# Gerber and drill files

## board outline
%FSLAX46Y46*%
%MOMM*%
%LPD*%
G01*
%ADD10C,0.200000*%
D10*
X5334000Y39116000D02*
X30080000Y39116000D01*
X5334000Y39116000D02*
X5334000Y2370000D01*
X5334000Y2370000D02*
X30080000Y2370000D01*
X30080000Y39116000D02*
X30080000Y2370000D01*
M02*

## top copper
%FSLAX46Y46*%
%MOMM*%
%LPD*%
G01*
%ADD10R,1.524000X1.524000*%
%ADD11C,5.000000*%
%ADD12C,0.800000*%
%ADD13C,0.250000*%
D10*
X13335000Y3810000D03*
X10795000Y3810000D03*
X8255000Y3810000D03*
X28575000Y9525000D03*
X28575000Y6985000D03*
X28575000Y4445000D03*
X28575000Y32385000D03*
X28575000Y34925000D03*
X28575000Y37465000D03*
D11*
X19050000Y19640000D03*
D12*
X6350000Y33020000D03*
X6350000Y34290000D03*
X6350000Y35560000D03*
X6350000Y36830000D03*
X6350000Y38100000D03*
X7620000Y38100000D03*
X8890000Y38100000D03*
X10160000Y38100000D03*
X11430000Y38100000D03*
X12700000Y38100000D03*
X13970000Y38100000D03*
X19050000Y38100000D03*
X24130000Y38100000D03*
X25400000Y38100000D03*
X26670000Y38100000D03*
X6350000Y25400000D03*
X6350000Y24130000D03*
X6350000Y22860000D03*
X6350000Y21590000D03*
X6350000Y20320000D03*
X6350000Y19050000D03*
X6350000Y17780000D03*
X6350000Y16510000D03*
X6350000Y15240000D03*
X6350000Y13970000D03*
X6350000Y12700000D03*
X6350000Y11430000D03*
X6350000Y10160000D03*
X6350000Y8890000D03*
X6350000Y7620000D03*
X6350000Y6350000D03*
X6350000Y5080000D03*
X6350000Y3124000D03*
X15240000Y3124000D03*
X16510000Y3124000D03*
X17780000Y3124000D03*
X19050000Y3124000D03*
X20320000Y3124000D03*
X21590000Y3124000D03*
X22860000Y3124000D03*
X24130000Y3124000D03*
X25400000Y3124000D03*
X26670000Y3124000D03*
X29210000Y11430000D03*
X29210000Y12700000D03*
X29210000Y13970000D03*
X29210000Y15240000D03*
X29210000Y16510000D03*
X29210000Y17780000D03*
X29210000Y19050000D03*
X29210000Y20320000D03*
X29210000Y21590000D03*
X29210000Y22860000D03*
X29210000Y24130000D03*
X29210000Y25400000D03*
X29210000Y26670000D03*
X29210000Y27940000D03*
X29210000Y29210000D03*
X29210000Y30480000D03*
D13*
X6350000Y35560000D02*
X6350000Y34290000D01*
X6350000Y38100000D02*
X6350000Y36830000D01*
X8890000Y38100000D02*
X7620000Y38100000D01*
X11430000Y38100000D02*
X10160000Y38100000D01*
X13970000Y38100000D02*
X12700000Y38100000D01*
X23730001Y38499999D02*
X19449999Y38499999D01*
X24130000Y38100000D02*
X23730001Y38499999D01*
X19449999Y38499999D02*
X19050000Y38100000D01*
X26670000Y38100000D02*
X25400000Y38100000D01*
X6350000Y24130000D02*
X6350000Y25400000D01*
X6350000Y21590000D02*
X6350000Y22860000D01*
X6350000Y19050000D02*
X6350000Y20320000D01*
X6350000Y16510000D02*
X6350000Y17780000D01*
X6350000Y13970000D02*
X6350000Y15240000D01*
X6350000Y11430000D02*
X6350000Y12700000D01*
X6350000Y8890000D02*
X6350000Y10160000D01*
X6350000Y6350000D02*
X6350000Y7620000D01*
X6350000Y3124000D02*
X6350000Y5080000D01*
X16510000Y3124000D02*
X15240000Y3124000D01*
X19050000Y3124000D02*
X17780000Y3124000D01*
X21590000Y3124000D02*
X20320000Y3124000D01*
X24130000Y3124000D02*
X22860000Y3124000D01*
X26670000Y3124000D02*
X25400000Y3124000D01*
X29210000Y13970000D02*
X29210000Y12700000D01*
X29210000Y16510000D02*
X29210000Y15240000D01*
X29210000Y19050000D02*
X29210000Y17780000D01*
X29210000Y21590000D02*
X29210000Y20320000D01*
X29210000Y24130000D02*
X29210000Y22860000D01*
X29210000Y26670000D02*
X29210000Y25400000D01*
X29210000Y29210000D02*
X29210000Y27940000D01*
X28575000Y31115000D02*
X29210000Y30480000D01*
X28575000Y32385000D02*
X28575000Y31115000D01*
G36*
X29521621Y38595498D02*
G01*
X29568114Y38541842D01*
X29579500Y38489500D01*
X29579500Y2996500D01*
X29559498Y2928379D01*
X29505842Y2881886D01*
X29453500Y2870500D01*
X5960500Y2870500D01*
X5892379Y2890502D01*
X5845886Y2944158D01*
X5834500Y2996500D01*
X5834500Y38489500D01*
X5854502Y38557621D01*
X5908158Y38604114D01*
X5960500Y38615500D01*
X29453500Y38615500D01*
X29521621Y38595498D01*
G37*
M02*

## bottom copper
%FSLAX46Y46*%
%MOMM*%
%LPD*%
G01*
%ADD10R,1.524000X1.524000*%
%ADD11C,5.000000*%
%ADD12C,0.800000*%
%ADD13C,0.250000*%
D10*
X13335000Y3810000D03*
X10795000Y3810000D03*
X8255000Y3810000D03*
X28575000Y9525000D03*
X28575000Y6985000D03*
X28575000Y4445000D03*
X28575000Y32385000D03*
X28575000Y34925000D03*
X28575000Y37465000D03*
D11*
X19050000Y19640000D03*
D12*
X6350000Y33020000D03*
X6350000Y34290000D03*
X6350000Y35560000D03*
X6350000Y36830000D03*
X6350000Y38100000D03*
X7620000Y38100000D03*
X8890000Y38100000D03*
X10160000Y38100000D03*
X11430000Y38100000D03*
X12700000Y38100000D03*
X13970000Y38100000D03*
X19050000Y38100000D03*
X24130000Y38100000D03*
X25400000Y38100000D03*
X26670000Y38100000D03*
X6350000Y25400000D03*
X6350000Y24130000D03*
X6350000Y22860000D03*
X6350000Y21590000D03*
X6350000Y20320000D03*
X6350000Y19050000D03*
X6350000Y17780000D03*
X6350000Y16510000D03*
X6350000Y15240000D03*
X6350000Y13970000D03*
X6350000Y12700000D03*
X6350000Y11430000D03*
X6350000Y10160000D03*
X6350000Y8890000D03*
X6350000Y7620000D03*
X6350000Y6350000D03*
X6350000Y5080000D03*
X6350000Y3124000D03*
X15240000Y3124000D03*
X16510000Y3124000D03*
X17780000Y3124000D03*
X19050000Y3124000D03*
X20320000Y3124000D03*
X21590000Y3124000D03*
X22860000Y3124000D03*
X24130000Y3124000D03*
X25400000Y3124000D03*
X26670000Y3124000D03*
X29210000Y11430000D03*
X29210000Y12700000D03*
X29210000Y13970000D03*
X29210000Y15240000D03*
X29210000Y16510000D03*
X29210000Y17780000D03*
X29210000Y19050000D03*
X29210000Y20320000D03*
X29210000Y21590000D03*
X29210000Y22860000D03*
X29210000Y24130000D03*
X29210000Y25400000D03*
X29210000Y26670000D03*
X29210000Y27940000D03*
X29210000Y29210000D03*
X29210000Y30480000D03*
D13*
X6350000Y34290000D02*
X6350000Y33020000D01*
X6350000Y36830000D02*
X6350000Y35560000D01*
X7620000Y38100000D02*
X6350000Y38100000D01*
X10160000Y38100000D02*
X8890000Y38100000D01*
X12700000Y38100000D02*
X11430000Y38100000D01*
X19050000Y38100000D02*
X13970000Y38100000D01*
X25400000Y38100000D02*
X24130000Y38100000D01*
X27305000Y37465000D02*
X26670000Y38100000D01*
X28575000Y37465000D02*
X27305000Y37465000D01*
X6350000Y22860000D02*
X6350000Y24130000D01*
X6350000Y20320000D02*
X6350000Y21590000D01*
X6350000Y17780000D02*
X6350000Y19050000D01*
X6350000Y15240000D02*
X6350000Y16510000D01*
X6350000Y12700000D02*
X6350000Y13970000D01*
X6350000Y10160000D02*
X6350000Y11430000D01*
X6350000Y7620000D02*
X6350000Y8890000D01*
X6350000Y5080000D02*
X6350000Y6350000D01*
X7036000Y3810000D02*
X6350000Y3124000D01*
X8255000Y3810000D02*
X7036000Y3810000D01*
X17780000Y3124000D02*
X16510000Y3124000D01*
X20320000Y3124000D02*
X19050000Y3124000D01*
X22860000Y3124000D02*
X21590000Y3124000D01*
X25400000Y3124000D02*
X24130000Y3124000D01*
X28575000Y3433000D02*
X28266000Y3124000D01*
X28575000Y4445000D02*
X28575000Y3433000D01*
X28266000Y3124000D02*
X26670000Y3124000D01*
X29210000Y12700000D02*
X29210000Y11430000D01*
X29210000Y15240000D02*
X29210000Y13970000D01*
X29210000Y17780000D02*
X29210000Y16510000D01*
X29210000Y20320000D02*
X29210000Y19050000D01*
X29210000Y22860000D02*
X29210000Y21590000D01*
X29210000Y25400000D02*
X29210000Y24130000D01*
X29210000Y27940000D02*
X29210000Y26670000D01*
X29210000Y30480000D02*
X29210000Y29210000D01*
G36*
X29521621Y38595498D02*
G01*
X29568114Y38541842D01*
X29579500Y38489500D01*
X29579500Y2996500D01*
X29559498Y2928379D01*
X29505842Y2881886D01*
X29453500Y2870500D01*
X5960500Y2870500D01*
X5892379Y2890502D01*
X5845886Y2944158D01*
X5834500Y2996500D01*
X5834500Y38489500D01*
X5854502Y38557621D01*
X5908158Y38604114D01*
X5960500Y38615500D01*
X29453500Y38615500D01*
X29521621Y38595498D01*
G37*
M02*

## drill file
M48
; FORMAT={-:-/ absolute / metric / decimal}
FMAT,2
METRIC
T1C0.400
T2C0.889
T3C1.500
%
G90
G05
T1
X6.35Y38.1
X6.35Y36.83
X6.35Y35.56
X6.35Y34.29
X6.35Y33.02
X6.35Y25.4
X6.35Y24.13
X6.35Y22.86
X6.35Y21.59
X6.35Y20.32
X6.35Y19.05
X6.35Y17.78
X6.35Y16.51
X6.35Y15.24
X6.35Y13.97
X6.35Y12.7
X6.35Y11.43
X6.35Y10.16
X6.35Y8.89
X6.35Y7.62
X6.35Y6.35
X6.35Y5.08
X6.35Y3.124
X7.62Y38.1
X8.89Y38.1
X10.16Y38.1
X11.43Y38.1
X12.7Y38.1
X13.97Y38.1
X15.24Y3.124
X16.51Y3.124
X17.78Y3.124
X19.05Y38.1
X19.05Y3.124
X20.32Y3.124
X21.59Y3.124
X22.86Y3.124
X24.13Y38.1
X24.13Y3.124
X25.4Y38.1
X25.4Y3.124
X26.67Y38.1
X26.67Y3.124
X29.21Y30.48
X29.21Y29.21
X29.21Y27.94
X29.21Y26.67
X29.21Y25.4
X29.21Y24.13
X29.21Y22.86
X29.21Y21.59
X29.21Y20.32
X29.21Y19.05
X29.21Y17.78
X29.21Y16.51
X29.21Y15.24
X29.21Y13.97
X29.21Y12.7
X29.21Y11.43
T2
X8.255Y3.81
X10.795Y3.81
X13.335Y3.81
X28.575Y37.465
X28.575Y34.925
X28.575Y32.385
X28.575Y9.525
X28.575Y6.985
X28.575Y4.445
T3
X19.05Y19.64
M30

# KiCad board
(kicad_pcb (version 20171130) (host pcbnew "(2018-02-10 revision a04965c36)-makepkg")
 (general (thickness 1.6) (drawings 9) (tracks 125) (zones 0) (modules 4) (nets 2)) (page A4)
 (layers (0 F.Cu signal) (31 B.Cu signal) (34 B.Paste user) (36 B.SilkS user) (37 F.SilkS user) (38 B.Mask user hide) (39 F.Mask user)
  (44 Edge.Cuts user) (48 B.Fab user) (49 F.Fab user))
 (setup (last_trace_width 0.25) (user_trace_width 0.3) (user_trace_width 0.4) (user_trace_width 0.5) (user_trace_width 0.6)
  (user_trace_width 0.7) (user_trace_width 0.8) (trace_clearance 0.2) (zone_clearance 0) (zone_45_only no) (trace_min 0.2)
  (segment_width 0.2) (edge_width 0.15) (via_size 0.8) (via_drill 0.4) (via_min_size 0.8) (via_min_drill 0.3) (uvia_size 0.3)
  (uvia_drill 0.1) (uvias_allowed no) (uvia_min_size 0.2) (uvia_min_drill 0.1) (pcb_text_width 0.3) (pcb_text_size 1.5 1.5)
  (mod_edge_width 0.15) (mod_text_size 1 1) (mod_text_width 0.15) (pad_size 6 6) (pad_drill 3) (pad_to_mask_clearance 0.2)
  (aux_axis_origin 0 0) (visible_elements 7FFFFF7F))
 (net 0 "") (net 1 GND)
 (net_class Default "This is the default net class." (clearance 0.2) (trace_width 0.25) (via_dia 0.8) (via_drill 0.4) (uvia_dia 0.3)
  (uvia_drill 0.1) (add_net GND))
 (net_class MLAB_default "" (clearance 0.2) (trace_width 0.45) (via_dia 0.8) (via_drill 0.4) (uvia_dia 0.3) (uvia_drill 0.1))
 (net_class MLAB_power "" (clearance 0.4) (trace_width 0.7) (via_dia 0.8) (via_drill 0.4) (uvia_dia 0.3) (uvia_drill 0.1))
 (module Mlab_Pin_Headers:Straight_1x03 (layer F.Cu) (at 10.795 -3.81 90)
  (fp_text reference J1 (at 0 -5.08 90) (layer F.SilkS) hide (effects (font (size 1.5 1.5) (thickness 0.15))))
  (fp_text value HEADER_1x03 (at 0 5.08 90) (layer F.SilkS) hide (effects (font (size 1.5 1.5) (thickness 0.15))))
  (pad 3 thru_hole rect (at 0 2.54 90) (size 1.524 1.524) (drill 0.889) (layers *.Cu *.Mask F.SilkS) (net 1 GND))
  (pad 2 thru_hole rect (at 0 0 90) (size 1.524 1.524) (drill 0.889) (layers *.Cu *.Mask F.SilkS) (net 1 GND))
  (pad 1 thru_hole rect (at 0 -2.54 90) (size 1.524 1.524) (drill 0.889) (layers *.Cu *.Mask F.SilkS) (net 1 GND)))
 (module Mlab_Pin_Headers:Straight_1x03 (layer F.Cu) (at 28.575 -6.985)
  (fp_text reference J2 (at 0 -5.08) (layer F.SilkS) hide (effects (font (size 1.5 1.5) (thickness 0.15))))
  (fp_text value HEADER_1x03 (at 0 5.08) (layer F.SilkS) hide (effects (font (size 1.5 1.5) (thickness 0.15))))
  (pad 1 thru_hole rect (at 0 -2.54) (size 1.524 1.524) (drill 0.889) (layers *.Cu *.Mask F.SilkS) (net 1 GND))
  (pad 2 thru_hole rect (at 0 0) (size 1.524 1.524) (drill 0.889) (layers *.Cu *.Mask F.SilkS) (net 1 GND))
  (pad 3 thru_hole rect (at 0 2.54) (size 1.524 1.524) (drill 0.889) (layers *.Cu *.Mask F.SilkS) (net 1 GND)))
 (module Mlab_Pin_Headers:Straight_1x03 (layer F.Cu) (at 28.575 -34.925)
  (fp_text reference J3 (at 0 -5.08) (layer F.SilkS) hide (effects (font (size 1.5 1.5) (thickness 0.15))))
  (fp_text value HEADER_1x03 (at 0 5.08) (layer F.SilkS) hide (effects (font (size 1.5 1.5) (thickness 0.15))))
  (pad 3 thru_hole rect (at 0 2.54) (size 1.524 1.524) (drill 0.889) (layers *.Cu *.Mask F.SilkS) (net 1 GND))
  (pad 2 thru_hole rect (at 0 0) (size 1.524 1.524) (drill 0.889) (layers *.Cu *.Mask F.SilkS) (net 1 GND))
  (pad 1 thru_hole rect (at 0 -2.54) (size 1.524 1.524) (drill 0.889) (layers *.Cu *.Mask F.SilkS) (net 1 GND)))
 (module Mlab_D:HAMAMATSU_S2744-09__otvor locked (layer F.Cu) (at 19.05 -5.2 270)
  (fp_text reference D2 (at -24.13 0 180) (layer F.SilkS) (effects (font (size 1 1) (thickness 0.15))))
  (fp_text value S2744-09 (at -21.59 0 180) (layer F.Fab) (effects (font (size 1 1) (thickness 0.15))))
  (pad 1 thru_hole circle (at -14.44 0 270) (size 5 5) (drill 1.5) (layers *.Cu *.Mask) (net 1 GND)))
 (gr_line (start 5.334 -39.116) (end 30.08 -39.116) (layer Edge.Cuts) (width 0.2))
 (gr_line (start 5.334 -39.116) (end 5.334 -2.37) (layer Edge.Cuts) (width 0.2))
 (gr_line (start 5.334 -2.37) (end 30.08 -2.37) (layer Edge.Cuts) (width 0.2))
 (gr_line (start 30.08 -39.116) (end 30.08 -2.37) (layer Edge.Cuts) (width 0.2))
 (segment (start 6.35 -34.29) (end 6.35 -33.02) (width 0.25) (layer B.Cu) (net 1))
 (via (at 6.35 -33.02) (size 0.8) (drill 0.4) (layers F.Cu B.Cu) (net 1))
 (segment (start 6.35 -35.56) (end 6.35 -34.29) (width 0.25) (layer F.Cu) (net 1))
 (via (at 6.35 -34.29) (size 0.8) (drill 0.4) (layers F.Cu B.Cu) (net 1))
 (segment (start 6.35 -36.83) (end 6.35 -35.56) (width 0.25) (layer B.Cu) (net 1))
 (via (at 6.35 -35.56) (size 0.8) (drill 0.4) (layers F.Cu B.Cu) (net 1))
 (segment (start 6.35 -38.1) (end 6.35 -36.83) (width 0.25) (layer F.Cu) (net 1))
 (via (at 6.35 -36.83) (size 0.8) (drill 0.4) (layers F.Cu B.Cu) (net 1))
 (segment (start 7.62 -38.1) (end 6.35 -38.1) (width 0.25) (layer B.Cu) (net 1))
 (via (at 6.35 -38.1) (size 0.8) (drill 0.4) (layers F.Cu B.Cu) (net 1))
 (segment (start 8.89 -38.1) (end 7.62 -38.1) (width 0.25) (layer F.Cu) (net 1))
 (via (at 7.62 -38.1) (size 0.8) (drill 0.4) (layers F.Cu B.Cu) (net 1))
 (segment (start 10.16 -38.1) (end 8.89 -38.1) (width 0.25) (layer B.Cu) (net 1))
 (via (at 8.89 -38.1) (size 0.8) (drill 0.4) (layers F.Cu B.Cu) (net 1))
 (segment (start 11.43 -38.1) (end 10.16 -38.1) (width 0.25) (layer F.Cu) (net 1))
 (via (at 10.16 -38.1) (size 0.8) (drill 0.4) (layers F.Cu B.Cu) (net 1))
 (segment (start 12.7 -38.1) (end 11.43 -38.1) (width 0.25) (layer B.Cu) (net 1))
 (via (at 11.43 -38.1) (size 0.8) (drill 0.4) (layers F.Cu B.Cu) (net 1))
 (segment (start 13.97 -38.1) (end 12.7 -38.1) (width 0.25) (layer F.Cu) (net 1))
 (via (at 12.7 -38.1) (size 0.8) (drill 0.4) (layers F.Cu B.Cu) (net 1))
 (segment (start 19.05 -38.1) (end 13.97 -38.1) (width 0.25) (layer B.Cu) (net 1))
 (via (at 13.97 -38.1) (size 0.8) (drill 0.4) (layers F.Cu B.Cu) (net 1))
 (segment (start 23.730001 -38.499999) (end 19.449999 -38.499999) (width 0.25) (layer F.Cu) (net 1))
 (segment (start 24.13 -38.1) (end 23.730001 -38.499999) (width 0.25) (layer F.Cu) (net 1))
 (segment (start 19.449999 -38.499999) (end 19.05 -38.1) (width 0.25) (layer F.Cu) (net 1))
 (via (at 19.05 -38.1) (size 0.8) (drill 0.4) (layers F.Cu B.Cu) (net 1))
 (segment (start 25.4 -38.1) (end 24.13 -38.1) (width 0.25) (layer B.Cu) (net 1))
 (via (at 24.13 -38.1) (size 0.8) (drill 0.4) (layers F.Cu B.Cu) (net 1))
 (segment (start 26.67 -38.1) (end 25.4 -38.1) (width 0.25) (layer F.Cu) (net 1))
 (via (at 25.4 -38.1) (size 0.8) (drill 0.4) (layers F.Cu B.Cu) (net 1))
 (segment (start 27.305 -37.465) (end 26.67 -38.1) (width 0.25) (layer B.Cu) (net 1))
 (segment (start 28.575 -37.465) (end 27.305 -37.465) (width 0.25) (layer B.Cu) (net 1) (status 10))
 (via (at 26.67 -38.1) (size 0.8) (drill 0.4) (layers F.Cu B.Cu) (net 1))
 (segment (start 6.35 -24.13) (end 6.35 -25.4) (width 0.25) (layer F.Cu) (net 1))
 (via (at 6.35 -25.4) (size 0.8) (drill 0.4) (layers F.Cu B.Cu) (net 1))
 (segment (start 6.35 -22.86) (end 6.35 -24.13) (width 0.25) (layer B.Cu) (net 1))
 (via (at 6.35 -24.13) (size 0.8) (drill 0.4) (layers F.Cu B.Cu) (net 1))
 (segment (start 6.35 -21.59) (end 6.35 -22.86) (width 0.25) (layer F.Cu) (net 1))
 (via (at 6.35 -22.86) (size 0.8) (drill 0.4) (layers F.Cu B.Cu) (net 1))
 (segment (start 6.35 -20.32) (end 6.35 -21.59) (width 0.25) (layer B.Cu) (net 1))
 (via (at 6.35 -21.59) (size 0.8) (drill 0.4) (layers F.Cu B.Cu) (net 1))
 (segment (start 6.35 -19.05) (end 6.35 -20.32) (width 0.25) (layer F.Cu) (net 1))
 (via (at 6.35 -20.32) (size 0.8) (drill 0.4) (layers F.Cu B.Cu) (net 1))
 (segment (start 6.35 -17.78) (end 6.35 -19.05) (width 0.25) (layer B.Cu) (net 1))
 (via (at 6.35 -19.05) (size 0.8) (drill 0.4) (layers F.Cu B.Cu) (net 1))
 (segment (start 6.35 -16.51) (end 6.35 -17.78) (width 0.25) (layer F.Cu) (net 1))
 (via (at 6.35 -17.78) (size 0.8) (drill 0.4) (layers F.Cu B.Cu) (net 1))
 (segment (start 6.35 -15.24) (end 6.35 -16.51) (width 0.25) (layer B.Cu) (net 1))
 (via (at 6.35 -16.51) (size 0.8) (drill 0.4) (layers F.Cu B.Cu) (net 1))
 (segment (start 6.35 -13.97) (end 6.35 -15.24) (width 0.25) (layer F.Cu) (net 1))
 (via (at 6.35 -15.24) (size 0.8) (drill 0.4) (layers F.Cu B.Cu) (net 1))
 (segment (start 6.35 -12.7) (end 6.35 -13.97) (width 0.25) (layer B.Cu) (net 1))
 (via (at 6.35 -13.97) (size 0.8) (drill 0.4) (layers F.Cu B.Cu) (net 1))
 (segment (start 6.35 -11.43) (end 6.35 -12.7) (width 0.25) (layer F.Cu) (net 1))
 (via (at 6.35 -12.7) (size 0.8) (drill 0.4) (layers F.Cu B.Cu) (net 1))
 (segment (start 6.35 -10.16) (end 6.35 -11.43) (width 0.25) (layer B.Cu) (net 1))
 (via (at 6.35 -11.43) (size 0.8) (drill 0.4) (layers F.Cu B.Cu) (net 1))
 (segment (start 6.35 -8.89) (end 6.35 -10.16) (width 0.25) (layer F.Cu) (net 1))
 (via (at 6.35 -10.16) (size 0.8) (drill 0.4) (layers F.Cu B.Cu) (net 1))
 (segment (start 6.35 -7.62) (end 6.35 -8.89) (width 0.25) (layer B.Cu) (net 1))
 (via (at 6.35 -8.89) (size 0.8) (drill 0.4) (layers F.Cu B.Cu) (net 1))
 (segment (start 6.35 -6.35) (end 6.35 -7.62) (width 0.25) (layer F.Cu) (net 1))
 (via (at 6.35 -7.62) (size 0.8) (drill 0.4) (layers F.Cu B.Cu) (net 1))
 (segment (start 6.35 -5.08) (end 6.35 -6.35) (width 0.25) (layer B.Cu) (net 1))
 (via (at 6.35 -6.35) (size 0.8) (drill 0.4) (layers F.Cu B.Cu) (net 1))
 (segment (start 6.35 -3.124) (end 6.35 -5.08) (width 0.25) (layer F.Cu) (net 1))
 (via (at 6.35 -5.08) (size 0.8) (drill 0.4) (layers F.Cu B.Cu) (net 1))
 (segment (start 7.036 -3.81) (end 6.35 -3.124) (width 0.25) (layer B.Cu) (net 1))
 (segment (start 8.255 -3.81) (end 7.036 -3.81) (width 0.25) (layer B.Cu) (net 1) (status 10))
 (via (at 6.35 -3.124) (size 0.8) (drill 0.4) (layers F.Cu B.Cu) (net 1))
 (segment (start 16.51 -3.124) (end 15.24 -3.124) (width 0.25) (layer F.Cu) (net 1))
 (via (at 15.24 -3.124) (size 0.8) (drill 0.4) (layers F.Cu B.Cu) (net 1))
 (segment (start 17.78 -3.124) (end 16.51 -3.124) (width 0.25) (layer B.Cu) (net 1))
 (via (at 16.51 -3.124) (size 0.8) (drill 0.4) (layers F.Cu B.Cu) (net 1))
 (segment (start 19.05 -3.124) (end 17.78 -3.124) (width 0.25) (layer F.Cu) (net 1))
 (via (at 17.78 -3.124) (size 0.8) (drill 0.4) (layers F.Cu B.Cu) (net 1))
 (segment (start 20.32 -3.124) (end 19.05 -3.124) (width 0.25) (layer B.Cu) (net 1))
 (via (at 19.05 -3.124) (size 0.8) (drill 0.4) (layers F.Cu B.Cu) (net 1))
 (segment (start 21.59 -3.124) (end 20.32 -3.124) (width 0.25) (layer F.Cu) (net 1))
 (via (at 20.32 -3.124) (size 0.8) (drill 0.4) (layers F.Cu B.Cu) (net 1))
 (segment (start 22.86 -3.124) (end 21.59 -3.124) (width 0.25) (layer B.Cu) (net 1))
 (via (at 21.59 -3.124) (size 0.8) (drill 0.4) (layers F.Cu B.Cu) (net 1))
 (segment (start 24.13 -3.124) (end 22.86 -3.124) (width 0.25) (layer F.Cu) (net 1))
 (via (at 22.86 -3.124) (size 0.8) (drill 0.4) (layers F.Cu B.Cu) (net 1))
 (segment (start 25.4 -3.124) (end 24.13 -3.124) (width 0.25) (layer B.Cu) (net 1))
 (via (at 24.13 -3.124) (size 0.8) (drill 0.4) (layers F.Cu B.Cu) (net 1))
 (segment (start 26.67 -3.124) (end 25.4 -3.124) (width 0.25) (layer F.Cu) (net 1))
 (via (at 25.4 -3.124) (size 0.8) (drill 0.4) (layers F.Cu B.Cu) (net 1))
 (segment (start 28.575 -3.433) (end 28.266 -3.124) (width 0.25) (layer B.Cu) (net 1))
 (segment (start 28.575 -4.445) (end 28.575 -3.433) (width 0.25) (layer B.Cu) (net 1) (status 10))
 (segment (start 28.266 -3.124) (end 26.67 -3.124) (width 0.25) (layer B.Cu) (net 1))
 (via (at 26.67 -3.124) (size 0.8) (drill 0.4) (layers F.Cu B.Cu) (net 1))
 (via (at 29.21 -11.43) (size 0.8) (drill 0.4) (layers F.Cu B.Cu) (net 1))
 (segment (start 29.21 -12.7) (end 29.21 -11.43) (width 0.25) (layer B.Cu) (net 1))
 (segment (start 29.21 -13.97) (end 29.21 -12.7) (width 0.25) (layer F.Cu) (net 1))
 (via (at 29.21 -12.7) (size 0.8) (drill 0.4) (layers F.Cu B.Cu) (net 1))
 (segment (start 29.21 -15.24) (end 29.21 -13.97) (width 0.25) (layer B.Cu) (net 1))
 (via (at 29.21 -13.97) (size 0.8) (drill 0.4) (layers F.Cu B.Cu) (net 1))
 (segment (start 29.21 -16.51) (end 29.21 -15.24) (width 0.25) (layer F.Cu) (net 1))
 (via (at 29.21 -15.24) (size 0.8) (drill 0.4) (layers F.Cu B.Cu) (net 1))
 (segment (start 29.21 -17.78) (end 29.21 -16.51) (width 0.25) (layer B.Cu) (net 1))
 (via (at 29.21 -16.51) (size 0.8) (drill 0.4) (layers F.Cu B.Cu) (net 1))
 (segment (start 29.21 -19.05) (end 29.21 -17.78) (width 0.25) (layer F.Cu) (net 1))
 (via (at 29.21 -17.78) (size 0.8) (drill 0.4) (layers F.Cu B.Cu) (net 1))
 (segment (start 29.21 -20.32) (end 29.21 -19.05) (width 0.25) (layer B.Cu) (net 1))
 (via (at 29.21 -19.05) (size 0.8) (drill 0.4) (layers F.Cu B.Cu) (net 1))
 (segment (start 29.21 -21.59) (end 29.21 -20.32) (width 0.25) (layer F.Cu) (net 1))
 (via (at 29.21 -20.32) (size 0.8) (drill 0.4) (layers F.Cu B.Cu) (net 1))
 (segment (start 29.21 -22.86) (end 29.21 -21.59) (width 0.25) (layer B.Cu) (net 1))
 (via (at 29.21 -21.59) (size 0.8) (drill 0.4) (layers F.Cu B.Cu) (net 1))
 (segment (start 29.21 -24.13) (end 29.21 -22.86) (width 0.25) (layer F.Cu) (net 1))
 (via (at 29.21 -22.86) (size 0.8) (drill 0.4) (layers F.Cu B.Cu) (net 1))
 (segment (start 29.21 -25.4) (end 29.21 -24.13) (width 0.25) (layer B.Cu) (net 1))
 (via (at 29.21 -24.13) (size 0.8) (drill 0.4) (layers F.Cu B.Cu) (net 1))
 (segment (start 29.21 -26.67) (end 29.21 -25.4) (width 0.25) (layer F.Cu) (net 1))
 (via (at 29.21 -25.4) (size 0.8) (drill 0.4) (layers F.Cu B.Cu) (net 1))
 (segment (start 29.21 -27.94) (end 29.21 -26.67) (width 0.25) (layer B.Cu) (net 1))
 (via (at 29.21 -26.67) (size 0.8) (drill 0.4) (layers F.Cu B.Cu) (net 1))
 (segment (start 29.21 -29.21) (end 29.21 -27.94) (width 0.25) (layer F.Cu) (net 1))
 (via (at 29.21 -27.94) (size 0.8) (drill 0.4) (layers F.Cu B.Cu) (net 1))
 (segment (start 29.21 -30.48) (end 29.21 -29.21) (width 0.25) (layer B.Cu) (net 1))
 (via (at 29.21 -29.21) (size 0.8) (drill 0.4) (layers F.Cu B.Cu) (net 1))
 (segment (start 28.575 -31.115) (end 29.21 -30.48) (width 0.25) (layer F.Cu) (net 1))
 (segment (start 28.575 -32.385) (end 28.575 -31.115) (width 0.25) (layer F.Cu) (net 1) (status 10))
 (via (at 29.21 -30.48) (size 0.8) (drill 0.4) (layers F.Cu B.Cu) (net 1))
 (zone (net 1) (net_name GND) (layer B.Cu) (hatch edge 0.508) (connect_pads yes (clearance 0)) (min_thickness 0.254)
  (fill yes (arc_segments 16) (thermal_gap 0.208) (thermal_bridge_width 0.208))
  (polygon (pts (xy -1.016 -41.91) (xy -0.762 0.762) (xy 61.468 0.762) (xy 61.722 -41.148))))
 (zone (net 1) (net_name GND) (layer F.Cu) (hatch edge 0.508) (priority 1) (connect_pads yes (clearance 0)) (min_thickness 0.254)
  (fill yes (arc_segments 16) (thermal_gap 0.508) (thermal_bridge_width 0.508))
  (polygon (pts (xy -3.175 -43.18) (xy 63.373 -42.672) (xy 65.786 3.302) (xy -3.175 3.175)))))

